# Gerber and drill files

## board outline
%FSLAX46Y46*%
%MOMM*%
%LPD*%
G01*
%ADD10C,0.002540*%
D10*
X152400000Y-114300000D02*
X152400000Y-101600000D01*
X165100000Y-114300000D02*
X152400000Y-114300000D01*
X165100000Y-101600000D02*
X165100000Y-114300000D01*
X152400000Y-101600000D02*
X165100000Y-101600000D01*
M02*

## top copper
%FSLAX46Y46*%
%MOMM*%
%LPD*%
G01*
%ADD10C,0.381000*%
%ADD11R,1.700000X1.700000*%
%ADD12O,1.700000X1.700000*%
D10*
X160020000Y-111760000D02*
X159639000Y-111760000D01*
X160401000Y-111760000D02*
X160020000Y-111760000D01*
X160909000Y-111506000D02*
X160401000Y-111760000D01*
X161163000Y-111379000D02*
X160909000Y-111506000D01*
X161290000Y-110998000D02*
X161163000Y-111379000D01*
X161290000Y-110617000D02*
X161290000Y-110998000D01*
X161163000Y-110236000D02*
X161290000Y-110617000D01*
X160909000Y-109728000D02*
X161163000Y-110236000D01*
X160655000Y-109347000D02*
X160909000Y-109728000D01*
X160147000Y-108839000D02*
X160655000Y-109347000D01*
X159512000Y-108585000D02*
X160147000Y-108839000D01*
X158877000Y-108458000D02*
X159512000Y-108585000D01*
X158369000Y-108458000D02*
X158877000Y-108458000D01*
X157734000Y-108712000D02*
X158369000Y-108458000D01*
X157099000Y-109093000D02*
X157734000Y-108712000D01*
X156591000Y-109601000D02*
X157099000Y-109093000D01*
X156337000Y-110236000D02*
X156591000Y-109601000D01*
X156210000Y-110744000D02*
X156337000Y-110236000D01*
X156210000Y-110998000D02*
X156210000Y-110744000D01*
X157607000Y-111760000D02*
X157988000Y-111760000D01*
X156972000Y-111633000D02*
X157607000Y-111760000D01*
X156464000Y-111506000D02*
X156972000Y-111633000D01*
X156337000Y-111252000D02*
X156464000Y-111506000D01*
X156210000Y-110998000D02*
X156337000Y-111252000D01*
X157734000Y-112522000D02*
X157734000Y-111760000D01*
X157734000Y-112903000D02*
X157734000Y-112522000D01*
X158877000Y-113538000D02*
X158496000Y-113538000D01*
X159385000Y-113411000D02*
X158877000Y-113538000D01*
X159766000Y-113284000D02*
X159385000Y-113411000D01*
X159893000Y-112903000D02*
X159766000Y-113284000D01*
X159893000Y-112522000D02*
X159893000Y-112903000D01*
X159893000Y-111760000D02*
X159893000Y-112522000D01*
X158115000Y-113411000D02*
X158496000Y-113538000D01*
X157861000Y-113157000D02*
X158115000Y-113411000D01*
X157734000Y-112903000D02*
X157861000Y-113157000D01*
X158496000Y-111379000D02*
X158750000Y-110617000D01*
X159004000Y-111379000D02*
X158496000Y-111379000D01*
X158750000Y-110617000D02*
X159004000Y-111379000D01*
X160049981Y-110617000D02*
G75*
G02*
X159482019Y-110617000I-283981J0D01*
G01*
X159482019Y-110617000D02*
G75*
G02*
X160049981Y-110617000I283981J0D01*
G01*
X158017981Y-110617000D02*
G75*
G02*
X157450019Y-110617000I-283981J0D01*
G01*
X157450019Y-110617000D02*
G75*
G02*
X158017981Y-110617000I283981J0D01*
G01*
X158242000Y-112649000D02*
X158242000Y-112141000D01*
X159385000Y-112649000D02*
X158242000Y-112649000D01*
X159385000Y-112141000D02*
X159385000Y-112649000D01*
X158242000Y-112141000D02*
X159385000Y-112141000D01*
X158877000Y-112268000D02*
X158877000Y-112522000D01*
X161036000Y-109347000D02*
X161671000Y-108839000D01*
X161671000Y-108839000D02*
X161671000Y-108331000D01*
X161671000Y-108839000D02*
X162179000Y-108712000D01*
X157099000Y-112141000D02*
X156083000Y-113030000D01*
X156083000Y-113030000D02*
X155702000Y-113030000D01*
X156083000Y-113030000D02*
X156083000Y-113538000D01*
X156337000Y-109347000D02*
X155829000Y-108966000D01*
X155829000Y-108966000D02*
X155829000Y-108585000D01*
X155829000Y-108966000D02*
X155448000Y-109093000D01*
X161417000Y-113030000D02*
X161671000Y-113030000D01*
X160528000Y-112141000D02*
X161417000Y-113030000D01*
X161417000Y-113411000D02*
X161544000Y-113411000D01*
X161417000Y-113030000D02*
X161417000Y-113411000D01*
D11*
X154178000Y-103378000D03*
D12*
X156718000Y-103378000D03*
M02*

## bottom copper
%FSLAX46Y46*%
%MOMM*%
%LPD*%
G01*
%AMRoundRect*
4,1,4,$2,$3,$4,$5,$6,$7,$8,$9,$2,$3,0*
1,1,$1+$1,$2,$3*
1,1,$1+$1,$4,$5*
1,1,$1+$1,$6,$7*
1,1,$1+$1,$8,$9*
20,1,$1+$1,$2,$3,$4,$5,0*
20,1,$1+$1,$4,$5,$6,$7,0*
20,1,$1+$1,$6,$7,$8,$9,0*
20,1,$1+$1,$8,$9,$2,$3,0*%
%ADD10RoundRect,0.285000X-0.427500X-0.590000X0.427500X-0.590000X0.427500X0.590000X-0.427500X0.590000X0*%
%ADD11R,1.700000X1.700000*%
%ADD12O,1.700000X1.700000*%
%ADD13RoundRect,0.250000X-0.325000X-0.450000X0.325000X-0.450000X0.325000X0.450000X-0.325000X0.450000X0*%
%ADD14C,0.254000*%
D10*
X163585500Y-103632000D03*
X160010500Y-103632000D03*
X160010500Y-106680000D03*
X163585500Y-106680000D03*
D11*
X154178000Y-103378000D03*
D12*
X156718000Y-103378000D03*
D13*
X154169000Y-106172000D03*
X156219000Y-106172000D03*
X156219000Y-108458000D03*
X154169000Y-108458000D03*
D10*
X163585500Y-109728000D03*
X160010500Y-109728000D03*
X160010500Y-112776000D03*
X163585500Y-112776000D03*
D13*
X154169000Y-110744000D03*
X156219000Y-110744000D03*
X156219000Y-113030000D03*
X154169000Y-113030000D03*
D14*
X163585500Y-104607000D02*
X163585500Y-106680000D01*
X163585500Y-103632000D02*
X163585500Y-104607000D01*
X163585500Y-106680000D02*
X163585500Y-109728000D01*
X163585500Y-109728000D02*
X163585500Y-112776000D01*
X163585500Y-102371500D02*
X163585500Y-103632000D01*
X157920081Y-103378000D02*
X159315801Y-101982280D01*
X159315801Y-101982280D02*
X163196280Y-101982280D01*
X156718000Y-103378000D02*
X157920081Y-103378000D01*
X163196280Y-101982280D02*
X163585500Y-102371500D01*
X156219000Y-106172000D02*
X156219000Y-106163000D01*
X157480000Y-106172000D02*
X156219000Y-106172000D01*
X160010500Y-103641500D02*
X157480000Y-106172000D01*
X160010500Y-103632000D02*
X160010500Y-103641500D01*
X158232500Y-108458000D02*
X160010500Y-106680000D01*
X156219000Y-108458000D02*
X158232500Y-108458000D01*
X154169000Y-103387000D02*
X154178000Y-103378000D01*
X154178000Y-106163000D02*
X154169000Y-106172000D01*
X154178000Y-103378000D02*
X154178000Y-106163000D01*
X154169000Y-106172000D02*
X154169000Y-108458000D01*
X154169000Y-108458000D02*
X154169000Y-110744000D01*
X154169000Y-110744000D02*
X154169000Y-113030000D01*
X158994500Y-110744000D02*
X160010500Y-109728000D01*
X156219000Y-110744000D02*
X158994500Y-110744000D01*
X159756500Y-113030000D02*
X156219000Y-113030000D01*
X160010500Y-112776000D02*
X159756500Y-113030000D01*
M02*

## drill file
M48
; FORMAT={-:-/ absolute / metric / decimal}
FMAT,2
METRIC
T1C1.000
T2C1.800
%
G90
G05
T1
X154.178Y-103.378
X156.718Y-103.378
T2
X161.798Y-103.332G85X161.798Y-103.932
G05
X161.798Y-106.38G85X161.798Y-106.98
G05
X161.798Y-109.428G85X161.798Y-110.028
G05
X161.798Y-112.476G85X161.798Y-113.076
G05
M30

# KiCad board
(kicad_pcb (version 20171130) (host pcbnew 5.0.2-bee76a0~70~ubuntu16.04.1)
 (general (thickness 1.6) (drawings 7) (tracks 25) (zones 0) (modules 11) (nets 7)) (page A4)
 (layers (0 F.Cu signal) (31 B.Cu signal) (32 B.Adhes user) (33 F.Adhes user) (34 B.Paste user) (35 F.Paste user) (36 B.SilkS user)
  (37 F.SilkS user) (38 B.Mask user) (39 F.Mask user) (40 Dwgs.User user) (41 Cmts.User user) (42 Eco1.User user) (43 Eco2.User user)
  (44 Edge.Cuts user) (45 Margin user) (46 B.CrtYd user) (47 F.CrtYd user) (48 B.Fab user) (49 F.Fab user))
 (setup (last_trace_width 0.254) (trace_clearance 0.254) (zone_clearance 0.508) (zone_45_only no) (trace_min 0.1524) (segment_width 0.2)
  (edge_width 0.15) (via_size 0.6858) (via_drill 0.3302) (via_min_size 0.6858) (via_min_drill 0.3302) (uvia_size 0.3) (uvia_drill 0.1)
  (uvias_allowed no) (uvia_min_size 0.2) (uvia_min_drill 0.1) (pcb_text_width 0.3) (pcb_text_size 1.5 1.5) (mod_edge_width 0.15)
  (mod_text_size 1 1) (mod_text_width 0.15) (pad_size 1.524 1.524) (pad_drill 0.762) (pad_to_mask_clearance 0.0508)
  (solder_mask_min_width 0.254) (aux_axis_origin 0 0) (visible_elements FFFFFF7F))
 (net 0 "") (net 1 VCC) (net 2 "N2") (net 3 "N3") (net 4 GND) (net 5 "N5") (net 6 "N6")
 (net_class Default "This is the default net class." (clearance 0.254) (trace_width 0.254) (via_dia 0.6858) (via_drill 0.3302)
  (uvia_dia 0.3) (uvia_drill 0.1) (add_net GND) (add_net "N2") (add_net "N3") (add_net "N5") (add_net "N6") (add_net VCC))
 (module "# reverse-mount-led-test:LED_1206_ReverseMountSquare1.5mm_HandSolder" (layer B.Cu) (at 161.798 103.632)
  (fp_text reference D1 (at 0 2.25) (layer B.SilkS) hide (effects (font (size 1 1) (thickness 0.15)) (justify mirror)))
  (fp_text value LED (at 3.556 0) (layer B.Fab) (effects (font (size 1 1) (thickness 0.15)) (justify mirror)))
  (pad "" np_thru_hole oval (at 0 0) (size 1.8 2.4) (drill oval 1.8 2.4) (layers *.Cu *.Mask))
  (pad 2 smd roundrect (at 1.7875 0) (size 1.425 1.75) (layers B.Cu B.Paste B.Mask) (roundrect_rratio 0.2) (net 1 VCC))
  (pad 1 smd roundrect (at -1.7875 0) (size 1.425 1.75) (layers B.Cu B.Paste B.Mask) (roundrect_rratio 0.2) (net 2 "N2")))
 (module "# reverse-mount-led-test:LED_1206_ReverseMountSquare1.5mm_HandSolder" (layer B.Cu) (at 161.798 106.68)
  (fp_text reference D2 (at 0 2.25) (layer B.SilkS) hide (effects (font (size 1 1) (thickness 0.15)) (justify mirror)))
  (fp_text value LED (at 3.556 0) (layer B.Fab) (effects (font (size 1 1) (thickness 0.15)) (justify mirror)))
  (pad 1 smd roundrect (at -1.7875 0) (size 1.425 1.75) (layers B.Cu B.Paste B.Mask) (roundrect_rratio 0.2) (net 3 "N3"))
  (pad 2 smd roundrect (at 1.7875 0) (size 1.425 1.75) (layers B.Cu B.Paste B.Mask) (roundrect_rratio 0.2) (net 1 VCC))
  (pad "" np_thru_hole oval (at 0 0) (size 1.8 2.4) (drill oval 1.8 2.4) (layers *.Cu *.Mask)))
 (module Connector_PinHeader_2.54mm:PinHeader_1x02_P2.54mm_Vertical (layer F.Cu) (at 154.178 103.378 90)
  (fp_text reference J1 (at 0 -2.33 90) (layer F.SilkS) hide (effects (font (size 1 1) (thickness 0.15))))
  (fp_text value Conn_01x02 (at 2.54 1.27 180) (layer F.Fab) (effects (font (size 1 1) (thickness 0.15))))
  (pad 1 thru_hole rect (at 0 0 90) (size 1.7 1.7) (drill 1) (layers *.Cu *.Mask) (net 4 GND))
  (pad 2 thru_hole oval (at 0 2.54 90) (size 1.7 1.7) (drill 1) (layers *.Cu *.Mask) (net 1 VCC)))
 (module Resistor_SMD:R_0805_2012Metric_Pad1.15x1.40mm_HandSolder (layer B.Cu) (at 155.194 106.172)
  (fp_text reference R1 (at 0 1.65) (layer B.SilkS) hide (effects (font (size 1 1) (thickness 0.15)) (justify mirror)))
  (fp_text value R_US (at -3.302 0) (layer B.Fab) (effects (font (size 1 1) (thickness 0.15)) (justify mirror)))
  (pad 1 smd roundrect (at -1.025 0) (size 1.15 1.4) (layers B.Cu B.Paste B.Mask) (roundrect_rratio 0.217391) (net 4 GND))
  (pad 2 smd roundrect (at 1.025 0) (size 1.15 1.4) (layers B.Cu B.Paste B.Mask) (roundrect_rratio 0.217391) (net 2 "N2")))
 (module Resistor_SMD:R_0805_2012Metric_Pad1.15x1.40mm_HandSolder (layer B.Cu) (at 155.194 108.458)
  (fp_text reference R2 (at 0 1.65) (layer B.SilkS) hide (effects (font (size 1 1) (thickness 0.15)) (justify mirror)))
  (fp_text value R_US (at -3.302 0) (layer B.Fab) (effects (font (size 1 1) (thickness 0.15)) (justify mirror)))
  (pad 2 smd roundrect (at 1.025 0) (size 1.15 1.4) (layers B.Cu B.Paste B.Mask) (roundrect_rratio 0.217391) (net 3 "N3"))
  (pad 1 smd roundrect (at -1.025 0) (size 1.15 1.4) (layers B.Cu B.Paste B.Mask) (roundrect_rratio 0.217391) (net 4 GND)))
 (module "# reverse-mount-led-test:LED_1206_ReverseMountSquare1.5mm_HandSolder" (layer B.Cu) (at 161.798 109.728)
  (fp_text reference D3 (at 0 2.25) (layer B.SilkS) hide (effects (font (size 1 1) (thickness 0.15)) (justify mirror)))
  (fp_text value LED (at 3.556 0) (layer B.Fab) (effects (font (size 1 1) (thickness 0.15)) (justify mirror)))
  (pad "" np_thru_hole oval (at 0 0) (size 1.8 2.4) (drill oval 1.8 2.4) (layers *.Cu *.Mask))
  (pad 2 smd roundrect (at 1.7875 0) (size 1.425 1.75) (layers B.Cu B.Paste B.Mask) (roundrect_rratio 0.2) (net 1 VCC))
  (pad 1 smd roundrect (at -1.7875 0) (size 1.425 1.75) (layers B.Cu B.Paste B.Mask) (roundrect_rratio 0.2) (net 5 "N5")))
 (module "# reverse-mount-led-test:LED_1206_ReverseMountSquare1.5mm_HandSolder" (layer B.Cu) (at 161.798 112.776)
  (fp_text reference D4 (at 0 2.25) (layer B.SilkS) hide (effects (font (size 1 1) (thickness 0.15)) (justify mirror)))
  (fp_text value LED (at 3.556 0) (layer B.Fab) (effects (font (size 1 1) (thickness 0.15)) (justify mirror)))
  (pad 1 smd roundrect (at -1.7875 0) (size 1.425 1.75) (layers B.Cu B.Paste B.Mask) (roundrect_rratio 0.2) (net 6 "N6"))
  (pad 2 smd roundrect (at 1.7875 0) (size 1.425 1.75) (layers B.Cu B.Paste B.Mask) (roundrect_rratio 0.2) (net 1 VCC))
  (pad "" np_thru_hole oval (at 0 0) (size 1.8 2.4) (drill oval 1.8 2.4) (layers *.Cu *.Mask)))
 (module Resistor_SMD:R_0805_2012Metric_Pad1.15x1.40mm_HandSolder (layer B.Cu) (at 155.194 110.744)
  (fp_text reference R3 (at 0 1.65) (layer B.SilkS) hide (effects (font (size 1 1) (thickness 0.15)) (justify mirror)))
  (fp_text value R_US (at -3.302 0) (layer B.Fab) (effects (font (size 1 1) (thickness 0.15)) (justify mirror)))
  (pad 1 smd roundrect (at -1.025 0) (size 1.15 1.4) (layers B.Cu B.Paste B.Mask) (roundrect_rratio 0.217391) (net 4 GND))
  (pad 2 smd roundrect (at 1.025 0) (size 1.15 1.4) (layers B.Cu B.Paste B.Mask) (roundrect_rratio 0.217391) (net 5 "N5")))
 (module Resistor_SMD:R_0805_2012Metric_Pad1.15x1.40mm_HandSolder (layer B.Cu) (at 155.194 113.03)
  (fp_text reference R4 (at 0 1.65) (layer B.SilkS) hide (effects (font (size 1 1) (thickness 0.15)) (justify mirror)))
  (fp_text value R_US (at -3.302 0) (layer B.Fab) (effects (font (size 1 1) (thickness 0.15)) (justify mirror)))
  (pad 2 smd roundrect (at 1.025 0) (size 1.15 1.4) (layers B.Cu B.Paste B.Mask) (roundrect_rratio 0.217391) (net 6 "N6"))
  (pad 1 smd roundrect (at -1.025 0) (size 1.15 1.4) (layers B.Cu B.Paste B.Mask) (roundrect_rratio 0.217391) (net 4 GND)))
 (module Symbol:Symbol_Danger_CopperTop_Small (layer F.Cu) (at 158.75 110.998)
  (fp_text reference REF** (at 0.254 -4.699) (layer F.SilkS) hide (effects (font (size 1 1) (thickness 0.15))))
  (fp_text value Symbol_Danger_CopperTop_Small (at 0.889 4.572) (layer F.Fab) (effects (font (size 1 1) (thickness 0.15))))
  (fp_line (start 1.27 0.762) (end 0.889 0.762) (layer F.Cu) (width 0.381))
  (fp_line (start 1.651 0.762) (end 1.27 0.762) (layer F.Cu) (width 0.381))
  (fp_line (start 2.159 0.508) (end 1.651 0.762) (layer F.Cu) (width 0.381))
  (fp_line (start 2.413 0.381) (end 2.159 0.508) (layer F.Cu) (width 0.381))
  (fp_line (start 2.54 0) (end 2.413 0.381) (layer F.Cu) (width 0.381))
  (fp_line (start 2.54 -0.381) (end 2.54 0) (layer F.Cu) (width 0.381))
  (fp_line (start 2.413 -0.762) (end 2.54 -0.381) (layer F.Cu) (width 0.381))
  (fp_line (start 2.159 -1.27) (end 2.413 -0.762) (layer F.Cu) (width 0.381))
  (fp_line (start 1.905 -1.651) (end 2.159 -1.27) (layer F.Cu) (width 0.381))
  (fp_line (start 1.397 -2.159) (end 1.905 -1.651) (layer F.Cu) (width 0.381))
  (fp_line (start 0.762 -2.413) (end 1.397 -2.159) (layer F.Cu) (width 0.381))
  (fp_line (start 0.127 -2.54) (end 0.762 -2.413) (layer F.Cu) (width 0.381))
  (fp_line (start -0.381 -2.54) (end 0.127 -2.54) (layer F.Cu) (width 0.381))
  (fp_line (start -1.016 -2.286) (end -0.381 -2.54) (layer F.Cu) (width 0.381))
  (fp_line (start -1.651 -1.905) (end -1.016 -2.286) (layer F.Cu) (width 0.381))
  (fp_line (start -2.159 -1.397) (end -1.651 -1.905) (layer F.Cu) (width 0.381))
  (fp_line (start -2.413 -0.762) (end -2.159 -1.397) (layer F.Cu) (width 0.381))
  (fp_line (start -2.54 -0.254) (end -2.413 -0.762) (layer F.Cu) (width 0.381))
  (fp_line (start -2.54 0) (end -2.54 -0.254) (layer F.Cu) (width 0.381))
  (fp_line (start -1.143 0.762) (end -0.762 0.762) (layer F.Cu) (width 0.381))
  (fp_line (start -1.778 0.635) (end -1.143 0.762) (layer F.Cu) (width 0.381))
  (fp_line (start -2.286 0.508) (end -1.778 0.635) (layer F.Cu) (width 0.381))
  (fp_line (start -2.413 0.254) (end -2.286 0.508) (layer F.Cu) (width 0.381))
  (fp_line (start -2.54 0) (end -2.413 0.254) (layer F.Cu) (width 0.381))
  (fp_line (start -1.016 1.524) (end -1.016 0.762) (layer F.Cu) (width 0.381))
  (fp_line (start -1.016 1.905) (end -1.016 1.524) (layer F.Cu) (width 0.381))
  (fp_line (start 0.127 2.54) (end -0.254 2.54) (layer F.Cu) (width 0.381))
  (fp_line (start 0.635 2.413) (end 0.127 2.54) (layer F.Cu) (width 0.381))
  (fp_line (start 1.016 2.286) (end 0.635 2.413) (layer F.Cu) (width 0.381))
  (fp_line (start 1.143 1.905) (end 1.016 2.286) (layer F.Cu) (width 0.381))
  (fp_line (start 1.143 1.524) (end 1.143 1.905) (layer F.Cu) (width 0.381))
  (fp_line (start 1.143 0.762) (end 1.143 1.524) (layer F.Cu) (width 0.381))
  (fp_line (start -0.635 2.413) (end -0.254 2.54) (layer F.Cu) (width 0.381))
  (fp_line (start -0.889 2.159) (end -0.635 2.413) (layer F.Cu) (width 0.381))
  (fp_line (start -1.016 1.905) (end -0.889 2.159) (layer F.Cu) (width 0.381))
  (fp_line (start -0.254 0.381) (end 0 -0.381) (layer F.Cu) (width 0.381))
  (fp_line (start 0.254 0.381) (end -0.254 0.381) (layer F.Cu) (width 0.381))
  (fp_line (start 0 -0.381) (end 0.254 0.381) (layer F.Cu) (width 0.381))
  (fp_circle (center 1.016 -0.381) (end 1.27 -0.254) (layer F.Cu) (width 0.381))
  (fp_circle (center -1.016 -0.381) (end -1.27 -0.254) (layer F.Cu) (width 0.381))
  (fp_line (start -0.508 1.651) (end -0.508 1.143) (layer F.Cu) (width 0.381))
  (fp_line (start 0.635 1.651) (end -0.508 1.651) (layer F.Cu) (width 0.381))
  (fp_line (start 0.635 1.143) (end 0.635 1.651) (layer F.Cu) (width 0.381))
  (fp_line (start -0.508 1.143) (end 0.635 1.143) (layer F.Cu) (width 0.381))
  (fp_line (start 0.127 1.27) (end 0.127 1.524) (layer F.Cu) (width 0.381))
  (fp_line (start 2.286 -1.651) (end 2.921 -2.159) (layer F.Cu) (width 0.381))
  (fp_line (start 2.921 -2.159) (end 2.921 -2.667) (layer F.Cu) (width 0.381))
  (fp_line (start 2.921 -2.159) (end 3.429 -2.286) (layer F.Cu) (width 0.381))
  (fp_line (start -1.651 1.143) (end -2.667 2.032) (layer F.Cu) (width 0.381))
  (fp_line (start -2.667 2.032) (end -3.048 2.032) (layer F.Cu) (width 0.381))
  (fp_line (start -2.667 2.032) (end -2.667 2.54) (layer F.Cu) (width 0.381))
  (fp_line (start -2.413 -1.651) (end -2.921 -2.032) (layer F.Cu) (width 0.381))
  (fp_line (start -2.921 -2.032) (end -2.921 -2.413) (layer F.Cu) (width 0.381))
  (fp_line (start -2.921 -2.032) (end -3.302 -1.905) (layer F.Cu) (width 0.381))
  (fp_line (start 2.667 2.032) (end 2.921 2.032) (layer F.Cu) (width 0.381))
  (fp_line (start 1.778 1.143) (end 2.667 2.032) (layer F.Cu) (width 0.381))
  (fp_line (start 2.667 2.413) (end 2.794 2.413) (layer F.Cu) (width 0.381))
  (fp_line (start 2.667 2.032) (end 2.667 2.413) (layer F.Cu) (width 0.381)))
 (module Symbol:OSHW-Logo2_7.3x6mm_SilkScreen (layer F.Cu) (at 160.782 105.156)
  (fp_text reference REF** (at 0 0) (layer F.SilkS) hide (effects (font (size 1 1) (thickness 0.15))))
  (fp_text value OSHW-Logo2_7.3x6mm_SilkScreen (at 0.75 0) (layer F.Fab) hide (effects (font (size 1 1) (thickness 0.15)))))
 (gr_line (start 152.4 114.3) (end 152.4 101.6) (layer Edge.Cuts) (width 0.00254))
 (gr_line (start 165.1 114.3) (end 152.4 114.3) (layer Edge.Cuts) (width 0.00254))
 (gr_line (start 165.1 101.6) (end 165.1 114.3) (layer Edge.Cuts) (width 0.00254))
 (gr_line (start 152.4 101.6) (end 165.1 101.6) (layer Edge.Cuts) (width 0.00254))
 (segment (start 163.5855 104.607) (end 163.5855 106.68) (width 0.254) (layer B.Cu) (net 1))
 (segment (start 163.5855 103.632) (end 163.5855 104.607) (width 0.254) (layer B.Cu) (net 1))
 (segment (start 163.5855 106.68) (end 163.5855 109.728) (width 0.254) (layer B.Cu) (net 1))
 (segment (start 163.5855 109.728) (end 163.5855 112.776) (width 0.254) (layer B.Cu) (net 1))
 (segment (start 163.5855 102.3715) (end 163.5855 103.632) (width 0.254) (layer B.Cu) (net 1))
 (segment (start 157.920081 103.378) (end 159.315801 101.98228) (width 0.254) (layer B.Cu) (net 1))
 (segment (start 159.315801 101.98228) (end 163.19628 101.98228) (width 0.254) (layer B.Cu) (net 1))
 (segment (start 156.718 103.378) (end 157.920081 103.378) (width 0.254) (layer B.Cu) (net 1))
 (segment (start 163.19628 101.98228) (end 163.5855 102.3715) (width 0.254) (layer B.Cu) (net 1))
 (segment (start 156.219 106.172) (end 156.219 106.163) (width 0.254) (layer B.Cu) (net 2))
 (segment (start 157.48 106.172) (end 156.219 106.172) (width 0.254) (layer B.Cu) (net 2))
 (segment (start 160.0105 103.6415) (end 157.48 106.172) (width 0.254) (layer B.Cu) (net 2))
 (segment (start 160.0105 103.632) (end 160.0105 103.6415) (width 0.254) (layer B.Cu) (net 2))
 (segment (start 158.2325 108.458) (end 160.0105 106.68) (width 0.254) (layer B.Cu) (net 3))
 (segment (start 156.219 108.458) (end 158.2325 108.458) (width 0.254) (layer B.Cu) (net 3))
 (segment (start 154.169 103.387) (end 154.178 103.378) (width 0.254) (layer B.Cu) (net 4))
 (segment (start 154.178 106.163) (end 154.169 106.172) (width 0.254) (layer B.Cu) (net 4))
 (segment (start 154.178 103.378) (end 154.178 106.163) (width 0.254) (layer B.Cu) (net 4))
 (segment (start 154.169 106.172) (end 154.169 108.458) (width 0.254) (layer B.Cu) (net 4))
 (segment (start 154.169 108.458) (end 154.169 110.744) (width 0.254) (layer B.Cu) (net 4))
 (segment (start 154.169 110.744) (end 154.169 113.03) (width 0.254) (layer B.Cu) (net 4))
 (segment (start 158.9945 110.744) (end 160.0105 109.728) (width 0.254) (layer B.Cu) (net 5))
 (segment (start 156.219 110.744) (end 158.9945 110.744) (width 0.254) (layer B.Cu) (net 5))
 (segment (start 159.7565 113.03) (end 156.219 113.03) (width 0.254) (layer B.Cu) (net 6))
 (segment (start 160.0105 112.776) (end 159.7565 113.03) (width 0.254) (layer B.Cu) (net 6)))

